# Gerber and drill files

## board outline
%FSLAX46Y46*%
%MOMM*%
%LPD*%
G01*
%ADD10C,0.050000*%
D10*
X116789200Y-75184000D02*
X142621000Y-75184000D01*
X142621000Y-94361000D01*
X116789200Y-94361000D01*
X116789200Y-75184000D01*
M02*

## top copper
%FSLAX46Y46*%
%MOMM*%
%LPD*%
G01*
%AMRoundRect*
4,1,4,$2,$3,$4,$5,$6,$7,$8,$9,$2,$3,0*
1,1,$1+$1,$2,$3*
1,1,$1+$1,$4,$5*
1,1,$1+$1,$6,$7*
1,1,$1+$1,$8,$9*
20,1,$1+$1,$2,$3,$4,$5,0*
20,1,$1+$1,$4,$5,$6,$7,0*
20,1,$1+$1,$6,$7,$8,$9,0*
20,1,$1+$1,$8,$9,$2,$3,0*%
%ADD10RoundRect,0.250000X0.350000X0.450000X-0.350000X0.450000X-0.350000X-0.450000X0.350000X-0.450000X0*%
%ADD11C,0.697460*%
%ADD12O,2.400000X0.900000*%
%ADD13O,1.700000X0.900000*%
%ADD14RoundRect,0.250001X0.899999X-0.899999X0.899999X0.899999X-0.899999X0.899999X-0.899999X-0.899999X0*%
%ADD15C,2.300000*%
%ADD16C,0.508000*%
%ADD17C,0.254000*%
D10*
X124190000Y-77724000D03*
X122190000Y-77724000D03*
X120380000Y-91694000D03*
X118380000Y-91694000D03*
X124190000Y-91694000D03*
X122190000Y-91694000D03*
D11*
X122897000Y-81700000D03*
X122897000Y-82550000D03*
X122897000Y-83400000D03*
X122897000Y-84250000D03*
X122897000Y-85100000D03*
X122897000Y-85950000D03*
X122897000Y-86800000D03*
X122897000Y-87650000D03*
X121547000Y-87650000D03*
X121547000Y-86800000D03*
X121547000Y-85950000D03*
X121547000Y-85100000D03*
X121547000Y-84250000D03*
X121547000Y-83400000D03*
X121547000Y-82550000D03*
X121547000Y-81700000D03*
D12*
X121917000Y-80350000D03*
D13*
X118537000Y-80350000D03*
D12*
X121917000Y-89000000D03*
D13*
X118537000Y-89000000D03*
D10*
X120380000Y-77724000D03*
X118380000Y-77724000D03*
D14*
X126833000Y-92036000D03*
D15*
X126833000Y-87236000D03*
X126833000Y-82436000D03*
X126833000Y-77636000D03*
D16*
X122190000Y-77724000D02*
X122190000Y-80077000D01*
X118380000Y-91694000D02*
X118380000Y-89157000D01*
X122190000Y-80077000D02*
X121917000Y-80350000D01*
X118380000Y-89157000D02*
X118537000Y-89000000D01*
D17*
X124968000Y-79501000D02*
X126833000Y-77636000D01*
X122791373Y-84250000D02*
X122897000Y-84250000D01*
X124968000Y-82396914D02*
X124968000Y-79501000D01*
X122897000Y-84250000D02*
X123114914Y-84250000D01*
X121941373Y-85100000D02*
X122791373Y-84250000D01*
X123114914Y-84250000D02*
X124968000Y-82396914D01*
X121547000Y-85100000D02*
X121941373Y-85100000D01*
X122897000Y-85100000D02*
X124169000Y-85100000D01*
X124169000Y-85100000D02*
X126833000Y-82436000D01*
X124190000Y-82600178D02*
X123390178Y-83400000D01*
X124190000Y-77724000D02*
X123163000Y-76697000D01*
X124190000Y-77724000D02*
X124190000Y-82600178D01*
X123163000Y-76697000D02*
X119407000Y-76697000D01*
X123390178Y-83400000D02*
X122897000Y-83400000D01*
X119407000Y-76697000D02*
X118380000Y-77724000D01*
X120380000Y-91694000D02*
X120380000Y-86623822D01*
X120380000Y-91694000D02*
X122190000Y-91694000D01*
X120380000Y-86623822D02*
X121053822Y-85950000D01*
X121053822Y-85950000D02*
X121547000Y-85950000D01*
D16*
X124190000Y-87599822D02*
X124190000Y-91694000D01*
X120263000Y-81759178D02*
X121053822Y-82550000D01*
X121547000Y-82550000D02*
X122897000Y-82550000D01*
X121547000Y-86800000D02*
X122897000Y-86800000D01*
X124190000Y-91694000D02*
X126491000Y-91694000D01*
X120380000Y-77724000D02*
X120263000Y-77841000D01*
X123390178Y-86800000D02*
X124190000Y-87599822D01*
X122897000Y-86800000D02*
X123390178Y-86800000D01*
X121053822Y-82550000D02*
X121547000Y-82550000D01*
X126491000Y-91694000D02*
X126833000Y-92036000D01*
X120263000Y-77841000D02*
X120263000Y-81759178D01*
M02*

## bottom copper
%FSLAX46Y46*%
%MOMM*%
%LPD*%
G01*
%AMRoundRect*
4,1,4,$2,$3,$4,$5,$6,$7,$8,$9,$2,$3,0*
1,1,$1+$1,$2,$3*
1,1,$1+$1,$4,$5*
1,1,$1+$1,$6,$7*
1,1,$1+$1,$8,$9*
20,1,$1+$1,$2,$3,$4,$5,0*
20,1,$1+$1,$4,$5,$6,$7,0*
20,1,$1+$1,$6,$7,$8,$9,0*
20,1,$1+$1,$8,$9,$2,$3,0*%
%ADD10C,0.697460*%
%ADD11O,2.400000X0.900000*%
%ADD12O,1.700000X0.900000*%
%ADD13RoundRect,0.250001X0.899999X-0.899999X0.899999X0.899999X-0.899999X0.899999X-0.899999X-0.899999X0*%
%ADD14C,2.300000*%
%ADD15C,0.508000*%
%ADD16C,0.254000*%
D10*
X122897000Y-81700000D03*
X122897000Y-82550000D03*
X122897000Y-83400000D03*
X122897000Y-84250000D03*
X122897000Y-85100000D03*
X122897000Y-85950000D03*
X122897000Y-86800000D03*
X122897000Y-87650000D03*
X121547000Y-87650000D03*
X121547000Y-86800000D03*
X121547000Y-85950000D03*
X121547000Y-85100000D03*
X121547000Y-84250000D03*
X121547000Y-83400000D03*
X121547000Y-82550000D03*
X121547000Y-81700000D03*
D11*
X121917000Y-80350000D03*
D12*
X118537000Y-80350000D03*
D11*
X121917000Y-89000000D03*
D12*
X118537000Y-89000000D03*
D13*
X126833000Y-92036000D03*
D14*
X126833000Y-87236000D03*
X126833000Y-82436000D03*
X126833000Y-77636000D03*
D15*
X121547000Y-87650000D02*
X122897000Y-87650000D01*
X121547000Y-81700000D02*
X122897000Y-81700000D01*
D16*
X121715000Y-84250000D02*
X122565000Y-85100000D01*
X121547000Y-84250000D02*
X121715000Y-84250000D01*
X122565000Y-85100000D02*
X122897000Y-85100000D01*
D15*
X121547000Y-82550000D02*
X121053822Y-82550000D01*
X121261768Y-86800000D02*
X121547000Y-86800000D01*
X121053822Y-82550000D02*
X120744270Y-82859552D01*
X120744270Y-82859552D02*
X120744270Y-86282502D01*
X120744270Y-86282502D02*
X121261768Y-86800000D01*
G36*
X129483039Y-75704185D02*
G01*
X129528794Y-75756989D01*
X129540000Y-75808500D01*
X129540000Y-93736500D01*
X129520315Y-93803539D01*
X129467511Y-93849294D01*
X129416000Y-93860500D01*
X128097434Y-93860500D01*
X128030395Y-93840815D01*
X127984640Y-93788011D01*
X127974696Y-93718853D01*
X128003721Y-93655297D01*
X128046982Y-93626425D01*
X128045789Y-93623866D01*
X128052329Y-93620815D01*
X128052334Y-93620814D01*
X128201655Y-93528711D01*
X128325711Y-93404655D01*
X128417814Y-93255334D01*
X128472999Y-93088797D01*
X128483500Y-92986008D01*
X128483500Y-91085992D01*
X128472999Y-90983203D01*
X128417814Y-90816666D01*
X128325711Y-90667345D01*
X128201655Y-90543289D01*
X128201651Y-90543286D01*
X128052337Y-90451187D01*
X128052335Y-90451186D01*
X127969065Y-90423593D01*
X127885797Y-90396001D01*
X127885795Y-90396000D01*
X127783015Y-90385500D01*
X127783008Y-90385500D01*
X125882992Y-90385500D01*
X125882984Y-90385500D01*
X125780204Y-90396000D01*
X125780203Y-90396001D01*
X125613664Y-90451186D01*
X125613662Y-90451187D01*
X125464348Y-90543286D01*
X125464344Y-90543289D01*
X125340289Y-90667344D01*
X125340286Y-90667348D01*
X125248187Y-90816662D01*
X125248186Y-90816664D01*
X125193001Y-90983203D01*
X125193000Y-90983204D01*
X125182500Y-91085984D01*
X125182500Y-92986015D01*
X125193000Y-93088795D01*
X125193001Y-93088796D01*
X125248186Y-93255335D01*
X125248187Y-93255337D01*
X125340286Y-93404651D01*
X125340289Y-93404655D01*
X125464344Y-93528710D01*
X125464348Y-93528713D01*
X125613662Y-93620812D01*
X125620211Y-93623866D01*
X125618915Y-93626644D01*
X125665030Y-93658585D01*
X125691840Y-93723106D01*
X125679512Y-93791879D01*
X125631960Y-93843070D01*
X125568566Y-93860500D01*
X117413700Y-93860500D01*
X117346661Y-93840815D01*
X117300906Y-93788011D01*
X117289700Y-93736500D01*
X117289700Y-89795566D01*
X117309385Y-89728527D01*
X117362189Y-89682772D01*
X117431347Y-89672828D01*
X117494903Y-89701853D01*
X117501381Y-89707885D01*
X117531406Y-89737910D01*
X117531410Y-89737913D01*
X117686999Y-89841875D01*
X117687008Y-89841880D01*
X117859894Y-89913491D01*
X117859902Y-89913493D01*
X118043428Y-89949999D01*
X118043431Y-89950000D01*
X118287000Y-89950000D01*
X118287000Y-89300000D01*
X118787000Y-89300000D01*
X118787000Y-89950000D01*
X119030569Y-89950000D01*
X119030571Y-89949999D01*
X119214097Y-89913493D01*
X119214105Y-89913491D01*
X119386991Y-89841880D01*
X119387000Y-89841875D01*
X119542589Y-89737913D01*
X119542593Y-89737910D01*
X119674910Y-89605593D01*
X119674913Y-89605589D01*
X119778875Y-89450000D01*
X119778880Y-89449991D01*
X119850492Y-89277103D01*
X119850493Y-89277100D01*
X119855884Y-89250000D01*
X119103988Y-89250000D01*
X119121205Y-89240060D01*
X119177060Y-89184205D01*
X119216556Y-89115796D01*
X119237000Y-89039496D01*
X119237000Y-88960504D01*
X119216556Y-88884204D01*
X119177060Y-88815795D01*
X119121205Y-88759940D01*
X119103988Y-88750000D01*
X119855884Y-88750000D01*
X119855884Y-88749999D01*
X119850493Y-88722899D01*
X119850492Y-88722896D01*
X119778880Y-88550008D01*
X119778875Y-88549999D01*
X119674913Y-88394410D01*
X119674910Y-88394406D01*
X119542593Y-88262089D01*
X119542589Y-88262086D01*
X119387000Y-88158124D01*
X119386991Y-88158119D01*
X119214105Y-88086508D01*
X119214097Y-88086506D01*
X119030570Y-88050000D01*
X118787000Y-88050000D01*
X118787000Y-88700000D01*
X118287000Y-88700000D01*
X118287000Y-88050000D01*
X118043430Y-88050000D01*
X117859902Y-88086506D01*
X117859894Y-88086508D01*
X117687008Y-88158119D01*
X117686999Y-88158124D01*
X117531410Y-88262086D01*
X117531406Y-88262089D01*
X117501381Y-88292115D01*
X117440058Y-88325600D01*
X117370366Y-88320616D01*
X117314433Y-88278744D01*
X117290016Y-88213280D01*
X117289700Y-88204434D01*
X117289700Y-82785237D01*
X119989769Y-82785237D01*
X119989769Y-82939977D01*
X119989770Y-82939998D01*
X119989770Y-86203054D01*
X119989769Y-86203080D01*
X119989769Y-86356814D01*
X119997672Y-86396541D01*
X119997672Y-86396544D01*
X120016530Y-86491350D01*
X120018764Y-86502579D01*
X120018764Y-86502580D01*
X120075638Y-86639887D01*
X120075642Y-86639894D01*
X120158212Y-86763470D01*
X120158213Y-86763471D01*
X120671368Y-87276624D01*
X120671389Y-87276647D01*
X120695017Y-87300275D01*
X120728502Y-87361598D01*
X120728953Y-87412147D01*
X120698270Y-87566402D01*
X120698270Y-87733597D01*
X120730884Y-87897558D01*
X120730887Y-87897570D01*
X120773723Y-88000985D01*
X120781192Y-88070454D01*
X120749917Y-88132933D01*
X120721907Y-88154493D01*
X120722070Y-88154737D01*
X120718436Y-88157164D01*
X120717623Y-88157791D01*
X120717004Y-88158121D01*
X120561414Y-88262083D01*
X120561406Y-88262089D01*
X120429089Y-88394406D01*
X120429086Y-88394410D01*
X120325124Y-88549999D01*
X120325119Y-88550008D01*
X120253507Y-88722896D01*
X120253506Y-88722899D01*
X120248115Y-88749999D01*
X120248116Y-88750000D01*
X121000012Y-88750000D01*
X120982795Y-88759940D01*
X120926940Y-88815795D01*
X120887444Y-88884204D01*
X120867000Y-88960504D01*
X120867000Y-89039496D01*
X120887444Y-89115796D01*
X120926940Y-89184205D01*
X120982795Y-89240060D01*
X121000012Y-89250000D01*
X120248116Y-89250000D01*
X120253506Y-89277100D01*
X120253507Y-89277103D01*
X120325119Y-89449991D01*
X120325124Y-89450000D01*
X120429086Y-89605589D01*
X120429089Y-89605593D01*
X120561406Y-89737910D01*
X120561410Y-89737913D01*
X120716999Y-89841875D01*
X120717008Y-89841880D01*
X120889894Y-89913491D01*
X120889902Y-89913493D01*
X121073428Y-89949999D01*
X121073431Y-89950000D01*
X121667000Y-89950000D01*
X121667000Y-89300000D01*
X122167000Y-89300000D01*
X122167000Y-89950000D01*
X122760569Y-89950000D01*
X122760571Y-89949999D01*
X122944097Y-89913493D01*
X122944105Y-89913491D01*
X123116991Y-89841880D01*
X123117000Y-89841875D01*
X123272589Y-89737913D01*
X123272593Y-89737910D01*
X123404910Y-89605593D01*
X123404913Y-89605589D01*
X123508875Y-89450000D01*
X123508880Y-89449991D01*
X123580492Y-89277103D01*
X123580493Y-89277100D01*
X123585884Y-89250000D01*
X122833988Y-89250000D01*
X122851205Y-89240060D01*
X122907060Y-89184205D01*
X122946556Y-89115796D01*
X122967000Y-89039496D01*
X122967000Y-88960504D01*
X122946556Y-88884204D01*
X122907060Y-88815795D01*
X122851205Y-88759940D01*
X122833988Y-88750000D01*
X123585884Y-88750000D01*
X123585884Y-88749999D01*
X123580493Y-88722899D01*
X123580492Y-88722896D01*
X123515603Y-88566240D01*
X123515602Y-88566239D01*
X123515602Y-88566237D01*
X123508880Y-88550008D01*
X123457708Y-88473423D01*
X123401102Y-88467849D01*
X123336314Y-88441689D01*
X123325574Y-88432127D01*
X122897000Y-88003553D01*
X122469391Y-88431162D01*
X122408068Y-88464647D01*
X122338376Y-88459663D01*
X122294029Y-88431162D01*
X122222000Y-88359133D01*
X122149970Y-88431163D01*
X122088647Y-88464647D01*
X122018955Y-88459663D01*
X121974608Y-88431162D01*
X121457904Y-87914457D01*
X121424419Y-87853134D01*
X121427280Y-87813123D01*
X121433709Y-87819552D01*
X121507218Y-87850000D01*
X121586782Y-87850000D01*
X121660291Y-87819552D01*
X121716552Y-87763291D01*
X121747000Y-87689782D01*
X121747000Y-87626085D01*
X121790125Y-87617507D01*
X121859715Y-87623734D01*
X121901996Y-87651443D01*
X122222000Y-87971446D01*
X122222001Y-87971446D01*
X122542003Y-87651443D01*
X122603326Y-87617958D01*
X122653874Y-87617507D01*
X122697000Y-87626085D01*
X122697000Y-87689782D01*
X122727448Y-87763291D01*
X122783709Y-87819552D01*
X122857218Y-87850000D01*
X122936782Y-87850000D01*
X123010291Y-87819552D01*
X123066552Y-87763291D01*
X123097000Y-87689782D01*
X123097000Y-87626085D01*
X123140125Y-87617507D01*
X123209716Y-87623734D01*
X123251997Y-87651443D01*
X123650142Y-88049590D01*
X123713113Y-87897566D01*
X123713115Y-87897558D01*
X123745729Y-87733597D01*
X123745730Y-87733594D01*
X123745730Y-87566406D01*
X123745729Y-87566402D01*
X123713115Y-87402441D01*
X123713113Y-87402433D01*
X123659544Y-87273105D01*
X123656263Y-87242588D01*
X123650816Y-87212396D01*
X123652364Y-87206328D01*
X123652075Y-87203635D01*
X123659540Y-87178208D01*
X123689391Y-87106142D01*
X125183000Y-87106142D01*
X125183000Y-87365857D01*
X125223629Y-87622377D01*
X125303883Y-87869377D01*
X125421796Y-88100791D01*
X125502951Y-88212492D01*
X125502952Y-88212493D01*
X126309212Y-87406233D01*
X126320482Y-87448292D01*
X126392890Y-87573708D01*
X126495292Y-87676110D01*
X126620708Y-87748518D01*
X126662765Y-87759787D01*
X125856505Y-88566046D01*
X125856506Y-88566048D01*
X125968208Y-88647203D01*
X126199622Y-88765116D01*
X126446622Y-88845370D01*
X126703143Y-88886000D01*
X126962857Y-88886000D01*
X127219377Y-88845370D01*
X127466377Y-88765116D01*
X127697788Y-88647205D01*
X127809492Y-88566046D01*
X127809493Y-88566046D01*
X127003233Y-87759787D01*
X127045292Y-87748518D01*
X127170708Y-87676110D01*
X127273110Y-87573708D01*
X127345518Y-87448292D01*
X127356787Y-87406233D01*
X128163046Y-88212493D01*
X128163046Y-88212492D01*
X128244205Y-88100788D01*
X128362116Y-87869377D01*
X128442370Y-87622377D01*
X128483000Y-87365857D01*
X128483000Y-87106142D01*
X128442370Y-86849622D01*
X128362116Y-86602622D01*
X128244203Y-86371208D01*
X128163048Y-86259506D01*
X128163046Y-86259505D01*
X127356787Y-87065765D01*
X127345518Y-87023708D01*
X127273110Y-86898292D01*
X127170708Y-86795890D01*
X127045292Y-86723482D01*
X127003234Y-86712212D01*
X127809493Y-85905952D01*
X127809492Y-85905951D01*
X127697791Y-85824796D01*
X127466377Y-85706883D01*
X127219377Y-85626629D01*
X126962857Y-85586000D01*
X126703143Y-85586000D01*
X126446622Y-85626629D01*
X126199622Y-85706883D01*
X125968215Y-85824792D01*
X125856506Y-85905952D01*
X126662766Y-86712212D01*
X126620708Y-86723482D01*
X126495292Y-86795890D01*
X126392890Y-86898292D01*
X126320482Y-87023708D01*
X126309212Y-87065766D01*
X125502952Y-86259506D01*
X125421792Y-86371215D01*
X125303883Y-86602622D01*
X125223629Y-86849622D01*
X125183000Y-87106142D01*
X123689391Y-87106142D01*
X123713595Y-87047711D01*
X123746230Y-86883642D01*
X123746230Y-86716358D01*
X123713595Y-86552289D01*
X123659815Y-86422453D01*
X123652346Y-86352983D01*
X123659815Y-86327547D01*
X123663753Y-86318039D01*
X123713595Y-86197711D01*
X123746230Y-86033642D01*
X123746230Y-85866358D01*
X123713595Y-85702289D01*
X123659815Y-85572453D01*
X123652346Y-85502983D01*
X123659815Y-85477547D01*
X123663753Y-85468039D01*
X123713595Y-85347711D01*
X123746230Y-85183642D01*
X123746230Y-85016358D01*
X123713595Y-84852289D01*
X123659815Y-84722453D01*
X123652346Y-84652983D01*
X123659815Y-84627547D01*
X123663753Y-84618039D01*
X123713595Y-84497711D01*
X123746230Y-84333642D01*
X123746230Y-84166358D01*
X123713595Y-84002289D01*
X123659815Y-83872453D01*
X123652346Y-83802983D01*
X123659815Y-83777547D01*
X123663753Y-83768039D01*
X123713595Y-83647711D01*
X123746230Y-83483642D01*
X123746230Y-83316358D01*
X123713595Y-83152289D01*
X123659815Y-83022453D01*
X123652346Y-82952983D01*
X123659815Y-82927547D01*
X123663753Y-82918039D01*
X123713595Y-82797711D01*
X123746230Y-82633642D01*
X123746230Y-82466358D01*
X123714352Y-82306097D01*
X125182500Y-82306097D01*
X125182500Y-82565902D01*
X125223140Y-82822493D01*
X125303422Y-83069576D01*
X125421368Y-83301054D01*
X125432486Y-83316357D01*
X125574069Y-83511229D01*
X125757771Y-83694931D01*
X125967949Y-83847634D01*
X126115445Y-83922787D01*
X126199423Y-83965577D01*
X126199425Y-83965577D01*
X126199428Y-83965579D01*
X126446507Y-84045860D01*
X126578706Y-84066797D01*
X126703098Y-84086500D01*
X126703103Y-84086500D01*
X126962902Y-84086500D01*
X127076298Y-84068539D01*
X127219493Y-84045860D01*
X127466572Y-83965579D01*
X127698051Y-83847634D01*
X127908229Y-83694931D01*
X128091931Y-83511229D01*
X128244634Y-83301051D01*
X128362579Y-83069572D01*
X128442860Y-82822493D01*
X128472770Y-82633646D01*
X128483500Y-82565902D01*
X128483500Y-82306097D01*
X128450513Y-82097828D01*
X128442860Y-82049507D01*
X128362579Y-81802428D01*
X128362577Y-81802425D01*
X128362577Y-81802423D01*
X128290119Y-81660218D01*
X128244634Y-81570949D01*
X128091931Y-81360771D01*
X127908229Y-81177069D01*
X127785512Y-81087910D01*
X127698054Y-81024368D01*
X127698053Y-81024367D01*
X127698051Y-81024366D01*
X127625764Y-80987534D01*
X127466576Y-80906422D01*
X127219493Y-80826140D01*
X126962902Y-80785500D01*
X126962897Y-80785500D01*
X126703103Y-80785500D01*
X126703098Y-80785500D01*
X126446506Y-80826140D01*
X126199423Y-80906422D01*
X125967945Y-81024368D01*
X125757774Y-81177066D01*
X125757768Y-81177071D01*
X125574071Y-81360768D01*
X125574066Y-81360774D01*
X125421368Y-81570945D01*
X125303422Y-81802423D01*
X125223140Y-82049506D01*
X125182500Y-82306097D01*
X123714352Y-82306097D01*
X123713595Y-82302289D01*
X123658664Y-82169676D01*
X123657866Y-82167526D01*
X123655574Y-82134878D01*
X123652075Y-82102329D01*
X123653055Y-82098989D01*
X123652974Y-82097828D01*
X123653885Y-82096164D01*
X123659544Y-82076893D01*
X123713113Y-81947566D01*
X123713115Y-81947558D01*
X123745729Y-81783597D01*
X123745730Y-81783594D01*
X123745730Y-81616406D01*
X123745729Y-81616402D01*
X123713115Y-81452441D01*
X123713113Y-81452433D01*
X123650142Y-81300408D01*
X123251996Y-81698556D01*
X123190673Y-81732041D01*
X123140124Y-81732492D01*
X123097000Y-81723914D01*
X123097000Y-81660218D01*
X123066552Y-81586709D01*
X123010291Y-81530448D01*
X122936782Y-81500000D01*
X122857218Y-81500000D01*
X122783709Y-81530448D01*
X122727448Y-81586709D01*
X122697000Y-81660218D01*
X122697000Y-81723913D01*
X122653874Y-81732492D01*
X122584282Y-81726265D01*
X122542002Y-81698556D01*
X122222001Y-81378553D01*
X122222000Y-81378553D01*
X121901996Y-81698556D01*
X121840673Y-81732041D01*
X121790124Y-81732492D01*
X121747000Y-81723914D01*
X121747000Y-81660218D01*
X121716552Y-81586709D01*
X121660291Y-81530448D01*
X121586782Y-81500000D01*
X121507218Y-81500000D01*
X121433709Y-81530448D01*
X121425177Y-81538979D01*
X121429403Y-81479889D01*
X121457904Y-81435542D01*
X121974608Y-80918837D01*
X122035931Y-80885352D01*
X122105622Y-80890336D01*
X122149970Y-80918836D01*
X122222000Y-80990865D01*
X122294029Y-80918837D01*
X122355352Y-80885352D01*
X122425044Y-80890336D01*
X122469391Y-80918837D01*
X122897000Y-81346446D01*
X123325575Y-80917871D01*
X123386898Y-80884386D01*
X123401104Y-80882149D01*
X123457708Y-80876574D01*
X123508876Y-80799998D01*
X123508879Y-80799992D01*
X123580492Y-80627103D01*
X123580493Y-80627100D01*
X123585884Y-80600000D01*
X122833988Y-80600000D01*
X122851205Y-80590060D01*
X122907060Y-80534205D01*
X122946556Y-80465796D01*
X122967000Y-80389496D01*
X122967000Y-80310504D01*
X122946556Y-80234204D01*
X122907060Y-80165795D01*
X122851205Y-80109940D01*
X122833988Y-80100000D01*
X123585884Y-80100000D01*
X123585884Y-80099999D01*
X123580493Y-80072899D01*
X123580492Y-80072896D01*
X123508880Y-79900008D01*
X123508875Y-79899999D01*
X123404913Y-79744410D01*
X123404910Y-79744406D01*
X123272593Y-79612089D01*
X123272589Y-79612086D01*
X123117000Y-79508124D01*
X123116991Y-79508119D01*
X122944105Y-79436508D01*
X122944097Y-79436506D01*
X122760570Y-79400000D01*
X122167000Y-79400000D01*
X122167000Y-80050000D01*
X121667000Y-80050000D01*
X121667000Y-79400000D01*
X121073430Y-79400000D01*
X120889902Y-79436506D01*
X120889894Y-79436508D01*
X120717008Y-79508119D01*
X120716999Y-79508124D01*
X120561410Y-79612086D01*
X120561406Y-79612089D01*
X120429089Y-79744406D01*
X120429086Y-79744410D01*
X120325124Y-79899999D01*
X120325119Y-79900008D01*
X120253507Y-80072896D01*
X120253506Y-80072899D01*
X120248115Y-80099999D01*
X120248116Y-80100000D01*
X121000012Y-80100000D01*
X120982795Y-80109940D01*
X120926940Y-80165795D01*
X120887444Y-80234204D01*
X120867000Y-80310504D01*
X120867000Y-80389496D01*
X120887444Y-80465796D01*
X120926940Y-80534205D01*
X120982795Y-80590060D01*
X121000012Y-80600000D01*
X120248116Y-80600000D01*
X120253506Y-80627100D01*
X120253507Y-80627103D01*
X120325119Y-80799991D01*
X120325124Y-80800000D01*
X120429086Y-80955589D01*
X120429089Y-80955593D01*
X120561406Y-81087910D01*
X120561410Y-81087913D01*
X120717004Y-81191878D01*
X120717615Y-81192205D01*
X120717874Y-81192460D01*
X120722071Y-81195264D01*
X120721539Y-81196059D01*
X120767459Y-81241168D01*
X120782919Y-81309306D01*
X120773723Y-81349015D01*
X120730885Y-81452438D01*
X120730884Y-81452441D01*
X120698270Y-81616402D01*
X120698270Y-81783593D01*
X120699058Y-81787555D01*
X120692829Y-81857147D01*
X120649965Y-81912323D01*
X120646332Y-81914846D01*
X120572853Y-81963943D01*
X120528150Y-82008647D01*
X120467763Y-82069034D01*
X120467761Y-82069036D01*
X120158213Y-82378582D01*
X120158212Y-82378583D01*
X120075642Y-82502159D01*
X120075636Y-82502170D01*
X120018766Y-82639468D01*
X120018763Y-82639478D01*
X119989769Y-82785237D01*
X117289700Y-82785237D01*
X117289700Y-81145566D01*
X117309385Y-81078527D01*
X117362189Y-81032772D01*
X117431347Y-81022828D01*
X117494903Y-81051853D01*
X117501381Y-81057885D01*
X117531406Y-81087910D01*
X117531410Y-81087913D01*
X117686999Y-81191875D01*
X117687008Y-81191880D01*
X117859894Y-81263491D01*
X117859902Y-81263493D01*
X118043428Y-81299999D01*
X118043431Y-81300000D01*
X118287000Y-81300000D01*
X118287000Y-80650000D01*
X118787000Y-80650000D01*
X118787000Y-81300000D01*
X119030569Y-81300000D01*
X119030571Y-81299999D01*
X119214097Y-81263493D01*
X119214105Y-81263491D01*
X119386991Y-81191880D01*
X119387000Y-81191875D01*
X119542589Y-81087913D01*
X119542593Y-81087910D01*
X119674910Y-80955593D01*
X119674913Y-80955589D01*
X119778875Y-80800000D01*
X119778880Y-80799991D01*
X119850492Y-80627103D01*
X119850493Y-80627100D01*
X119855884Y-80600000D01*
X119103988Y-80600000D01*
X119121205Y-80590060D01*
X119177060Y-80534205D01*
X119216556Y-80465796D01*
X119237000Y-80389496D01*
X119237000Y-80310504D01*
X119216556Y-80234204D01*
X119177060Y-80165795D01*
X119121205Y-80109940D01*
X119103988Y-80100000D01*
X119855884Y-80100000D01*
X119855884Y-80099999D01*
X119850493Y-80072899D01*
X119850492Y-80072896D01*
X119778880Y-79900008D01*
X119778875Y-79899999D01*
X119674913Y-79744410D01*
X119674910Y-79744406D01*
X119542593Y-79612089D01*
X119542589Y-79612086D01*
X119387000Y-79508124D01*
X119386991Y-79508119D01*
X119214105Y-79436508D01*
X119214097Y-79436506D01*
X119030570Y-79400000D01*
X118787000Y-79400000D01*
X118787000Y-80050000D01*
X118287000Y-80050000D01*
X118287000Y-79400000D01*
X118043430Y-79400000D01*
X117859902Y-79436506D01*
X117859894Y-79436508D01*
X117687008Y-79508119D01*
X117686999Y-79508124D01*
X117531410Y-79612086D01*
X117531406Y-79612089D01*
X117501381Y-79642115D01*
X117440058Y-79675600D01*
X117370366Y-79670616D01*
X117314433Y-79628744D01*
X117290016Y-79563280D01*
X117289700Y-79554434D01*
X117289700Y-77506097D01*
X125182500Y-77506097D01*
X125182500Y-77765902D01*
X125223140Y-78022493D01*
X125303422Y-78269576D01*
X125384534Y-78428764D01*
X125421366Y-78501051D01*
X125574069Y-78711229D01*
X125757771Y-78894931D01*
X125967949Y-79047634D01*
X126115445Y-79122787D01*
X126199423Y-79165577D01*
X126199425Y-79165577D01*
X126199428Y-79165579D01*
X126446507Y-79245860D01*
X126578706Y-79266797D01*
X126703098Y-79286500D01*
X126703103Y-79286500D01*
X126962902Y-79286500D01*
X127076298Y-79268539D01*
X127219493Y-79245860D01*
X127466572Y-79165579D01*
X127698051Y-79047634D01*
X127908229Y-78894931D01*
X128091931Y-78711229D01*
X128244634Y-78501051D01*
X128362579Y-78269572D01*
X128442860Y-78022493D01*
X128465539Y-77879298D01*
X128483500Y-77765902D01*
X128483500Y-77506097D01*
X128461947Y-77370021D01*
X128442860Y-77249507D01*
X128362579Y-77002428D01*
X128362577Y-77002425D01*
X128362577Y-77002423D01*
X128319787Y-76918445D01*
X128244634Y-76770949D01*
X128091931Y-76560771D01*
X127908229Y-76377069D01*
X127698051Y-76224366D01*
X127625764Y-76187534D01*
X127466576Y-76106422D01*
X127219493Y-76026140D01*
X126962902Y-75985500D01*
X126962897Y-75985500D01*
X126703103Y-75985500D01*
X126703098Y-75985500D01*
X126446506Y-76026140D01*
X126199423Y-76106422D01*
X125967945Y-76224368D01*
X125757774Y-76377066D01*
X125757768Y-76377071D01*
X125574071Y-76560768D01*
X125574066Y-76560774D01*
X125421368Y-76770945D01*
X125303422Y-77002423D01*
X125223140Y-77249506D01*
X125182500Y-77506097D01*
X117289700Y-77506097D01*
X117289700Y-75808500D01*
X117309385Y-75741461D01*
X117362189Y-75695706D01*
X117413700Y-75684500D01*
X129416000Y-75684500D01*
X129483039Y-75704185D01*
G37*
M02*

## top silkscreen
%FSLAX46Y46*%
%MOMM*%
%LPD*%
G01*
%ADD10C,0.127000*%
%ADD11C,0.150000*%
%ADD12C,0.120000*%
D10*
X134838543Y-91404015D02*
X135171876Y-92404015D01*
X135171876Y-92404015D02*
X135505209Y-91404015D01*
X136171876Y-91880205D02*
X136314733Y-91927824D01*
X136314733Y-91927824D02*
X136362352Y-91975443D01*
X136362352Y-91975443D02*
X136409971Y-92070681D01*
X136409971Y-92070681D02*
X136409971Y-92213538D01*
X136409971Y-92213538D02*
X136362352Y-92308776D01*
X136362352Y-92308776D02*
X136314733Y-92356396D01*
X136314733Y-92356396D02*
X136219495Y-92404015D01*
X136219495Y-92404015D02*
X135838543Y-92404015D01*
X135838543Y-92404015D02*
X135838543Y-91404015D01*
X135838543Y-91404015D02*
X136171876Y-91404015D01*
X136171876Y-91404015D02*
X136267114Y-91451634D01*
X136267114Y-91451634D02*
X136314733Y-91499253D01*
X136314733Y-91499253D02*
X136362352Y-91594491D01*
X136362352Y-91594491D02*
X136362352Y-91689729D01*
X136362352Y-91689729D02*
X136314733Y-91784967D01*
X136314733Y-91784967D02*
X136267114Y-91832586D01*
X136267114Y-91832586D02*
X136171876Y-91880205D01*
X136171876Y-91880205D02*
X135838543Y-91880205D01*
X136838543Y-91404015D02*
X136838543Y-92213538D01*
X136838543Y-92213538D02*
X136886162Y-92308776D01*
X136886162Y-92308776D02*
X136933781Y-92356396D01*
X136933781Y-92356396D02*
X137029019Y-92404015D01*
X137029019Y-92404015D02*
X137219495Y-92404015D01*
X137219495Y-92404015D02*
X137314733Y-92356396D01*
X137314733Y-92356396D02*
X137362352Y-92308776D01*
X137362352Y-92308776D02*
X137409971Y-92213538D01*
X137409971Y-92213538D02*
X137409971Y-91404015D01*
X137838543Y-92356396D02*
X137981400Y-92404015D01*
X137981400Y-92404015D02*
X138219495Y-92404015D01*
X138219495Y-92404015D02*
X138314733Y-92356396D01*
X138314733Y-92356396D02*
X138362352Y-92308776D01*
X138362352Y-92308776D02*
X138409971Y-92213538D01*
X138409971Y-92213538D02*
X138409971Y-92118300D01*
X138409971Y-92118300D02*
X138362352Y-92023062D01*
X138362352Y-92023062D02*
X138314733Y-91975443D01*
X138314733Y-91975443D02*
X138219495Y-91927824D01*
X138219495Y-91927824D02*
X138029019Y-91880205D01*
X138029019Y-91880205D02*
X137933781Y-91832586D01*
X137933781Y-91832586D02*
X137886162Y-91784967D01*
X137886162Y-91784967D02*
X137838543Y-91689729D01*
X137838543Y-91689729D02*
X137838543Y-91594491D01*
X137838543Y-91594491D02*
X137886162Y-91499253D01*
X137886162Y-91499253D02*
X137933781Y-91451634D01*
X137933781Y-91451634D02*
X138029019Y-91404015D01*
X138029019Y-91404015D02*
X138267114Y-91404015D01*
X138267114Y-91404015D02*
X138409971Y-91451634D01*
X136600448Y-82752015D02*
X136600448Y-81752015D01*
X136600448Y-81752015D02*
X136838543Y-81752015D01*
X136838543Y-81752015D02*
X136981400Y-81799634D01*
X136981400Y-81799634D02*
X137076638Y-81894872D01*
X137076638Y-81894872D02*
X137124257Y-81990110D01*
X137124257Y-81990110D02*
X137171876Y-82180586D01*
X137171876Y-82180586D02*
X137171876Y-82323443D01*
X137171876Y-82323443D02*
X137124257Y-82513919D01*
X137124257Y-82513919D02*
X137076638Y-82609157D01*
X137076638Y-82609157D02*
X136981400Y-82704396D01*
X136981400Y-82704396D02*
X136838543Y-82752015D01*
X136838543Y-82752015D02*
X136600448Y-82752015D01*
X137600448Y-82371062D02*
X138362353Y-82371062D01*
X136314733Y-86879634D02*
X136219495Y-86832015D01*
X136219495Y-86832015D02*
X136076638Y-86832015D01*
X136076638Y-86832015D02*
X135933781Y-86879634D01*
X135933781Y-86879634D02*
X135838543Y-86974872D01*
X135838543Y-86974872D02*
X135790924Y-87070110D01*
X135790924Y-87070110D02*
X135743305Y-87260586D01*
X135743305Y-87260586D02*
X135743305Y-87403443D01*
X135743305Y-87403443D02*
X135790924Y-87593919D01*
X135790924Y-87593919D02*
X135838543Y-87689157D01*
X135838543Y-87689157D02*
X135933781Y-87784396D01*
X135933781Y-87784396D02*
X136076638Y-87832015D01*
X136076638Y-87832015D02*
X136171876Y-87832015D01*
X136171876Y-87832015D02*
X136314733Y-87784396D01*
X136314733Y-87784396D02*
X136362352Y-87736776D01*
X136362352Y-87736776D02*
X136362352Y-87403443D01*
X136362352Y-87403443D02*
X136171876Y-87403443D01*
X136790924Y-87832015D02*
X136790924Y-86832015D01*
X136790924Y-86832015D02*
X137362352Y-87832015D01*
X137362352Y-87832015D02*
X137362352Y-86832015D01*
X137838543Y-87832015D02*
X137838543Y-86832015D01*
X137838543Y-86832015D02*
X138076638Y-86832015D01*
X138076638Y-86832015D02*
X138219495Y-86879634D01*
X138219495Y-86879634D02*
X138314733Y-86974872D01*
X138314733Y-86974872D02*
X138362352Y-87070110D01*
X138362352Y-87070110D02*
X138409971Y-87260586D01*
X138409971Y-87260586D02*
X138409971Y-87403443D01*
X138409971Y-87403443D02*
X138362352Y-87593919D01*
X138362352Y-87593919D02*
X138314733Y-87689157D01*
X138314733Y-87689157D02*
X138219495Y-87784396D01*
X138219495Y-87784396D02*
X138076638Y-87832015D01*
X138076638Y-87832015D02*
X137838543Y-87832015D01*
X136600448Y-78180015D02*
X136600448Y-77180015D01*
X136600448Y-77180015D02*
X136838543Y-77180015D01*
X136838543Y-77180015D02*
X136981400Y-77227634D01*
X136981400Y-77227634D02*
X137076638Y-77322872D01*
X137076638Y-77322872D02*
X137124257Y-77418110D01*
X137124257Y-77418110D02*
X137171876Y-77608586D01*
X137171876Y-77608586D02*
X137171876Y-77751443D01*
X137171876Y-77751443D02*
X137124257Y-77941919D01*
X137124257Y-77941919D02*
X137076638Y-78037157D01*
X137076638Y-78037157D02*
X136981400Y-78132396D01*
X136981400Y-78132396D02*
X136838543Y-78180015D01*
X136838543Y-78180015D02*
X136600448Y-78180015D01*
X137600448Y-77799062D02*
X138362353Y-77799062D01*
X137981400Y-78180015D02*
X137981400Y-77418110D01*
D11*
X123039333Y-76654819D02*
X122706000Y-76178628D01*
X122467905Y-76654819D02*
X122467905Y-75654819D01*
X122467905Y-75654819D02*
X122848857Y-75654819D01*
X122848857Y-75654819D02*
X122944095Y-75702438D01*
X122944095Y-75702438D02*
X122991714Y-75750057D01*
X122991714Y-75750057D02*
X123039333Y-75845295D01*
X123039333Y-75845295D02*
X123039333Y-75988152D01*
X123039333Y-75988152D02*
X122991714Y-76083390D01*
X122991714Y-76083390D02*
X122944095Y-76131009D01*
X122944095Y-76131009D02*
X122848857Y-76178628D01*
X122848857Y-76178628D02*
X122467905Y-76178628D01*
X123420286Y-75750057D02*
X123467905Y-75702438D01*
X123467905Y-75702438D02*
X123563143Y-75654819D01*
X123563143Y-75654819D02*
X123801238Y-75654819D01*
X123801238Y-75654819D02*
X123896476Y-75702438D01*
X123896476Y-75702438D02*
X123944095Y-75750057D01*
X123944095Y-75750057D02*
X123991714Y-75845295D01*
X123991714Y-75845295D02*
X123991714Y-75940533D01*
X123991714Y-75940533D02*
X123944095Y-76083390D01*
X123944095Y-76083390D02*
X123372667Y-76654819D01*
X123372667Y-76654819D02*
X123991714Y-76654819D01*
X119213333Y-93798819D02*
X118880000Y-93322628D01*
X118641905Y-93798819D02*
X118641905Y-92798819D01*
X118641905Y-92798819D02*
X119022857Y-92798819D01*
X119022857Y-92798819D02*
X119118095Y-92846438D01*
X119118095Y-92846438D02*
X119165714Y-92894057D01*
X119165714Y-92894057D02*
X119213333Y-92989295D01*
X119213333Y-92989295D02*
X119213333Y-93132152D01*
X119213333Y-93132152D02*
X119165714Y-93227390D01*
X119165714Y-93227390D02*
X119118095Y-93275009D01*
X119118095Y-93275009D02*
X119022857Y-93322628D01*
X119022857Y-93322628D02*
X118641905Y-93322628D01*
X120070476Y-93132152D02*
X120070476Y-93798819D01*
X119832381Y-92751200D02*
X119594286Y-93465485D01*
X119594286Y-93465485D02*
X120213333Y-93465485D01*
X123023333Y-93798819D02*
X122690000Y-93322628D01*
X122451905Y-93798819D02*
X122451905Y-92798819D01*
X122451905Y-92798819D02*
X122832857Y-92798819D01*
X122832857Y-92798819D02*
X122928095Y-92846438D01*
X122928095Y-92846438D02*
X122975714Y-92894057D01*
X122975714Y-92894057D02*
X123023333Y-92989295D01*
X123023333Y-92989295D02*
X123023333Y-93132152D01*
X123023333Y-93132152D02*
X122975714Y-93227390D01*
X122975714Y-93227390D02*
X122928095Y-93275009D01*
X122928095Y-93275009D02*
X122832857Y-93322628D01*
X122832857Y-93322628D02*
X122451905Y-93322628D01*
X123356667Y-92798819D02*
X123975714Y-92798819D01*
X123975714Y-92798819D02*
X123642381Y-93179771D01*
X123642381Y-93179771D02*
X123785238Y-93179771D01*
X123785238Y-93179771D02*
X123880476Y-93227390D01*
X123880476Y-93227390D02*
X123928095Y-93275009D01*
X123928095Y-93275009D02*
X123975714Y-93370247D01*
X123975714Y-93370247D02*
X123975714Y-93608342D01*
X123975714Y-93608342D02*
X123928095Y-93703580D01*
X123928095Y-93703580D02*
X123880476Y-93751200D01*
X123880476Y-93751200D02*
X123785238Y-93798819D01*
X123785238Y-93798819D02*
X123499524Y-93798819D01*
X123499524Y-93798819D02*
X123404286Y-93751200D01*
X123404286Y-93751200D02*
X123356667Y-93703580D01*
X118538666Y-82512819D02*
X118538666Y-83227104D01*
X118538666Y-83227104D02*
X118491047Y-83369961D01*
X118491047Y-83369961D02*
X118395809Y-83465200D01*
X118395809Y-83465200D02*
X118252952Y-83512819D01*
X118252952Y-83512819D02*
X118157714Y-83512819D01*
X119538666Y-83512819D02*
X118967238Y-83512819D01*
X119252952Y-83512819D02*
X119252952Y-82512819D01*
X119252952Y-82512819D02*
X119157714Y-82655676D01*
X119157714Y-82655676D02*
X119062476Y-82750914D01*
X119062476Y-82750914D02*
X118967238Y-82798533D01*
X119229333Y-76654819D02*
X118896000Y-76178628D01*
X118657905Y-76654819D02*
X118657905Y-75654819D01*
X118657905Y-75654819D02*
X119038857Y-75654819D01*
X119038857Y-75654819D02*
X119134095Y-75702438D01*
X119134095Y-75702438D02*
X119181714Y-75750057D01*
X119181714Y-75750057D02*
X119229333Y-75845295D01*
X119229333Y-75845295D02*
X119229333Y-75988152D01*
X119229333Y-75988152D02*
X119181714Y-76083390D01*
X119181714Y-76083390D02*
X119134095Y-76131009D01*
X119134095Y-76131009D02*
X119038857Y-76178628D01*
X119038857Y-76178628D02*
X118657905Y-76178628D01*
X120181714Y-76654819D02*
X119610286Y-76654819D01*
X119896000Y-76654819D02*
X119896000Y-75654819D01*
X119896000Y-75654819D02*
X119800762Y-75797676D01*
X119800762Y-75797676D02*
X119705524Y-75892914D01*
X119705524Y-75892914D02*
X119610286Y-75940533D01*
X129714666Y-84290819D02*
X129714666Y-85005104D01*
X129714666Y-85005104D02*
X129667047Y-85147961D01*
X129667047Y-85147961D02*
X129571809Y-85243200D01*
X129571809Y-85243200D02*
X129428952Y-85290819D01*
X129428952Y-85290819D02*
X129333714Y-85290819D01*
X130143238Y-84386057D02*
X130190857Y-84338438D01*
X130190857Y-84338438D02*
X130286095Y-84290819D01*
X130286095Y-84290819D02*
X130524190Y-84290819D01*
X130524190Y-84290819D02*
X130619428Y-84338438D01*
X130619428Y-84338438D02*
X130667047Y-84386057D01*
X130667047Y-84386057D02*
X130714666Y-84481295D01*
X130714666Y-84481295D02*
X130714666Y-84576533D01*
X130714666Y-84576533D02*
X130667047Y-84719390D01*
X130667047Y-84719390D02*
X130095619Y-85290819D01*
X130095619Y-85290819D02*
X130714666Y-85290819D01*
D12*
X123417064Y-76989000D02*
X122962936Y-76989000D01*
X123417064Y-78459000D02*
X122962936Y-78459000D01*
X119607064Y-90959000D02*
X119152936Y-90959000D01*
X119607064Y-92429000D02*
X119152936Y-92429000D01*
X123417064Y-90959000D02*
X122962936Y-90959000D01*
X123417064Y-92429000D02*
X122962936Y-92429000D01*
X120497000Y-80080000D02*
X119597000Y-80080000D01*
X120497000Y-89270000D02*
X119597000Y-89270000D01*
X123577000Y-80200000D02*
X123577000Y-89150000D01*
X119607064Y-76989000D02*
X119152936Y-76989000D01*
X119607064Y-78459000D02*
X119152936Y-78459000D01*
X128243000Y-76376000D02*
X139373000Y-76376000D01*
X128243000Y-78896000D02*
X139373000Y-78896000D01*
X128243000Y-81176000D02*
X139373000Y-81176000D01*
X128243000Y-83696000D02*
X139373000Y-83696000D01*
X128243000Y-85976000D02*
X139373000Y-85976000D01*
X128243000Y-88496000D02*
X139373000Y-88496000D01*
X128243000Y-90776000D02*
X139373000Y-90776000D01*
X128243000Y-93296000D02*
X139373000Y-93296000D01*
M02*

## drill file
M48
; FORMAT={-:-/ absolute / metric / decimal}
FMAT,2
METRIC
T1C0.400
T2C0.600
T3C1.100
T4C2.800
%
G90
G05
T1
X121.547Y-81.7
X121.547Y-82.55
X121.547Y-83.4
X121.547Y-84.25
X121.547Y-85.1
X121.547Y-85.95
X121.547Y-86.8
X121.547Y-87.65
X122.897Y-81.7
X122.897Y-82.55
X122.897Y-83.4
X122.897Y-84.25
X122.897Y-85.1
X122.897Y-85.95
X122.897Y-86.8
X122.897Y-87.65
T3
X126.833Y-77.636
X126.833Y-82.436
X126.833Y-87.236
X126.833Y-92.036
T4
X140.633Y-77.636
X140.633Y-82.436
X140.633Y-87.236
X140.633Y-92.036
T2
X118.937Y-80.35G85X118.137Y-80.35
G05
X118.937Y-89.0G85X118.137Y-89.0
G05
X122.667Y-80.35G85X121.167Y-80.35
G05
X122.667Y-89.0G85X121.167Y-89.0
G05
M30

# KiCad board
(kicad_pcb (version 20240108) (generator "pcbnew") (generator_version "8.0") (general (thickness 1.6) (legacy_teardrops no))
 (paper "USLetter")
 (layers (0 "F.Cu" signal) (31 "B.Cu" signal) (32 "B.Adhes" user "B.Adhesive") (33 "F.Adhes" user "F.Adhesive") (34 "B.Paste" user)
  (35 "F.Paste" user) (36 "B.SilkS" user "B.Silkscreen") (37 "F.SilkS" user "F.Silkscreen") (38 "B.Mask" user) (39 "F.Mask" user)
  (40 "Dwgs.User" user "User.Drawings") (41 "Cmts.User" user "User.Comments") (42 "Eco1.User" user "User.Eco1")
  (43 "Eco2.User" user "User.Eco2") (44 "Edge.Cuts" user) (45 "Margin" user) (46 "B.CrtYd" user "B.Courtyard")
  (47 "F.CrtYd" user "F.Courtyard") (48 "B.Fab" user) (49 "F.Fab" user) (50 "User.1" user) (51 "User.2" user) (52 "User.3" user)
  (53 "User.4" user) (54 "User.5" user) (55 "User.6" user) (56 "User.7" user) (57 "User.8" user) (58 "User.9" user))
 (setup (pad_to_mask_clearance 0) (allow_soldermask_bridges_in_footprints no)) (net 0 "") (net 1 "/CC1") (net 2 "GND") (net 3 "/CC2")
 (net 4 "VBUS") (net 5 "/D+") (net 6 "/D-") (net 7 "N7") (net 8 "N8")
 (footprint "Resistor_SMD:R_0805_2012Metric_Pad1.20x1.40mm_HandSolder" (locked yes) (layer "F.Cu") (at 123.19 77.724 180)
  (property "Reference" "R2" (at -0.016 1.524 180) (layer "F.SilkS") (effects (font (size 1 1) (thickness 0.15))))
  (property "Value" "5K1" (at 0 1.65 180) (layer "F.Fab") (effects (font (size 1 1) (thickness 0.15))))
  (fp_line (start -0.227064 0.735) (end 0.227064 0.735) (stroke (width 0.12) (type solid)) (layer "F.SilkS"))
  (fp_line (start -0.227064 -0.735) (end 0.227064 -0.735) (stroke (width 0.12) (type solid)) (layer "F.SilkS"))
  (pad "1" smd roundrect (at -1 0 180) (size 1.2 1.4) (layers "F.Cu" "F.Paste" "F.Mask") (roundrect_rratio 0.208333) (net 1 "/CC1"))
  (pad "2" smd roundrect (at 1 0 180) (size 1.2 1.4) (layers "F.Cu" "F.Paste" "F.Mask") (roundrect_rratio 0.208333) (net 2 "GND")))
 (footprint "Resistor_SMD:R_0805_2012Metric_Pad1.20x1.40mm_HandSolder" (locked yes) (layer "F.Cu") (at 119.38 91.694 180)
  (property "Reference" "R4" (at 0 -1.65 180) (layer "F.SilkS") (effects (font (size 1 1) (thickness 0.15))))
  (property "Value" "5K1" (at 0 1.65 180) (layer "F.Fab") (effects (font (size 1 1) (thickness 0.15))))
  (fp_line (start -0.227064 0.735) (end 0.227064 0.735) (stroke (width 0.12) (type solid)) (layer "F.SilkS"))
  (fp_line (start -0.227064 -0.735) (end 0.227064 -0.735) (stroke (width 0.12) (type solid)) (layer "F.SilkS"))
  (pad "1" smd roundrect (at -1 0 180) (size 1.2 1.4) (layers "F.Cu" "F.Paste" "F.Mask") (roundrect_rratio 0.208333) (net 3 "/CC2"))
  (pad "2" smd roundrect (at 1 0 180) (size 1.2 1.4) (layers "F.Cu" "F.Paste" "F.Mask") (roundrect_rratio 0.208333) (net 2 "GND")))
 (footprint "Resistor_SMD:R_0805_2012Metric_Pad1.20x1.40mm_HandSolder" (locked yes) (layer "F.Cu") (at 123.19 91.694 180)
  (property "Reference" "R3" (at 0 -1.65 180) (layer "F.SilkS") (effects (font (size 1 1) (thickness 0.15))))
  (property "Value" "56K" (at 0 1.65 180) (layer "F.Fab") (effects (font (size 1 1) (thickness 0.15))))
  (fp_line (start -0.227064 0.735) (end 0.227064 0.735) (stroke (width 0.12) (type solid)) (layer "F.SilkS"))
  (fp_line (start -0.227064 -0.735) (end 0.227064 -0.735) (stroke (width 0.12) (type solid)) (layer "F.SilkS"))
  (pad "1" smd roundrect (at -1 0 180) (size 1.2 1.4) (layers "F.Cu" "F.Paste" "F.Mask") (roundrect_rratio 0.208333) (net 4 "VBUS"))
  (pad "2" smd roundrect (at 1 0 180) (size 1.2 1.4) (layers "F.Cu" "F.Paste" "F.Mask") (roundrect_rratio 0.208333) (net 3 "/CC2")))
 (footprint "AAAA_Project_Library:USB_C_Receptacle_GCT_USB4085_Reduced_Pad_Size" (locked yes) (layer "F.Cu") (at 122.897 81.7 -90)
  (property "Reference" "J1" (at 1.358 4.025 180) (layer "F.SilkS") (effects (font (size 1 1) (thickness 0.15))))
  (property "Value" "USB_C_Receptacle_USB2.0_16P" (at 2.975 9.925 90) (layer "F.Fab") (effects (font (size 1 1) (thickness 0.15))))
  (fp_line (start -1.62 2.4) (end -1.62 3.3) (stroke (width 0.12) (type solid)) (layer "F.SilkS"))
  (fp_line (start 7.57 2.4) (end 7.57 3.3) (stroke (width 0.12) (type solid)) (layer "F.SilkS"))
  (fp_line (start -1.5 -0.68) (end 7.45 -0.68) (stroke (width 0.12) (type solid)) (layer "F.SilkS"))
  (pad "A1" thru_hole circle (at 0 0 270) (size 0.69746 0.69746) (drill 0.4) (layers "*.Cu" "*.Mask") (remove_unused_layers no)
   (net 2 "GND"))
  (pad "A4" thru_hole circle (at 0.85 0 270) (size 0.69746 0.69746) (drill 0.4) (layers "*.Cu" "*.Mask") (remove_unused_layers no)
   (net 4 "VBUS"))
  (pad "A5" thru_hole circle (at 1.7 0 270) (size 0.69746 0.69746) (drill 0.4) (layers "*.Cu" "*.Mask") (remove_unused_layers no)
   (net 1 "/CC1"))
  (pad "A6" thru_hole circle (at 2.55 0 270) (size 0.69746 0.69746) (drill 0.4) (layers "*.Cu" "*.Mask") (remove_unused_layers no)
   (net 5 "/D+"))
  (pad "A7" thru_hole circle (at 3.4 0 270) (size 0.69746 0.69746) (drill 0.4) (layers "*.Cu" "*.Mask") (remove_unused_layers no)
   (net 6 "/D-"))
  (pad "A8" thru_hole circle (at 4.25 0 270) (size 0.69746 0.69746) (drill 0.4) (layers "*.Cu" "*.Mask") (remove_unused_layers no)
   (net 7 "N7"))
  (pad "A9" thru_hole circle (at 5.1 0 270) (size 0.69746 0.69746) (drill 0.4) (layers "*.Cu" "*.Mask") (remove_unused_layers no)
   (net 4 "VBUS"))
  (pad "A12" thru_hole circle (at 5.95 0 270) (size 0.69746 0.69746) (drill 0.4) (layers "*.Cu" "*.Mask") (remove_unused_layers no)
   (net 2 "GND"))
  (pad "B1" thru_hole circle (at 5.95 1.35 270) (size 0.69746 0.69746) (drill 0.4) (layers "*.Cu" "*.Mask") (remove_unused_layers no)
   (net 2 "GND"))
  (pad "B4" thru_hole circle (at 5.1 1.35 270) (size 0.69746 0.69746) (drill 0.4) (layers "*.Cu" "*.Mask") (remove_unused_layers no)
   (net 4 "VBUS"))
  (pad "B5" thru_hole circle (at 4.25 1.35 270) (size 0.69746 0.69746) (drill 0.4) (layers "*.Cu" "*.Mask") (remove_unused_layers no)
   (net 3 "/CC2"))
  (pad "B6" thru_hole circle (at 3.4 1.35 270) (size 0.69746 0.69746) (drill 0.4) (layers "*.Cu" "*.Mask") (remove_unused_layers no)
   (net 5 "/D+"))
  (pad "B7" thru_hole circle (at 2.55 1.35 270) (size 0.69746 0.69746) (drill 0.4) (layers "*.Cu" "*.Mask") (remove_unused_layers no)
   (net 6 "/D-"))
  (pad "B8" thru_hole circle (at 1.7 1.35 270) (size 0.69746 0.69746) (drill 0.4) (layers "*.Cu" "*.Mask") (remove_unused_layers no)
   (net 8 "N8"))
  (pad "B9" thru_hole circle (at 0.85 1.35 270) (size 0.69746 0.69746) (drill 0.4) (layers "*.Cu" "*.Mask") (remove_unused_layers no)
   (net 4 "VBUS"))
  (pad "B12" thru_hole circle (at 0 1.35 270) (size 0.69746 0.69746) (drill 0.4) (layers "*.Cu" "*.Mask") (remove_unused_layers no)
   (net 2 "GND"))
  (pad "S1" thru_hole oval (at -1.35 0.98 270) (size 0.9 2.4) (drill oval 0.6 2.1) (layers "*.Cu" "*.Mask") (remove_unused_layers no)
   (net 2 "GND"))
  (pad "S1" thru_hole oval (at -1.35 4.36 270) (size 0.9 1.7) (drill oval 0.6 1.4) (layers "*.Cu" "*.Mask") (remove_unused_layers no)
   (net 2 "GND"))
  (pad "S1" thru_hole oval (at 7.3 0.98 270) (size 0.9 2.4) (drill oval 0.6 2.1) (layers "*.Cu" "*.Mask") (remove_unused_layers no)
   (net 2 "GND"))
  (pad "S1" thru_hole oval (at 7.3 4.36 270) (size 0.9 1.7) (drill oval 0.6 1.4) (layers "*.Cu" "*.Mask") (remove_unused_layers no)
   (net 2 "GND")))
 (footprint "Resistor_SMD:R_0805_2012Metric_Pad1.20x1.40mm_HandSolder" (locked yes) (layer "F.Cu") (at 119.38 77.724 180)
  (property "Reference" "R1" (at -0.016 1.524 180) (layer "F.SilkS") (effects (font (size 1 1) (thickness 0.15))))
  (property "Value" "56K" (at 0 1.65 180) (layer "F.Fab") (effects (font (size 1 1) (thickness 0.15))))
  (fp_line (start -0.227064 0.735) (end 0.227064 0.735) (stroke (width 0.12) (type solid)) (layer "F.SilkS"))
  (fp_line (start -0.227064 -0.735) (end 0.227064 -0.735) (stroke (width 0.12) (type solid)) (layer "F.SilkS"))
  (pad "1" smd roundrect (at -1 0 180) (size 1.2 1.4) (layers "F.Cu" "F.Paste" "F.Mask") (roundrect_rratio 0.208333) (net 4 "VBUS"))
  (pad "2" smd roundrect (at 1 0 180) (size 1.2 1.4) (layers "F.Cu" "F.Paste" "F.Mask") (roundrect_rratio 0.208333) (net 1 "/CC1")))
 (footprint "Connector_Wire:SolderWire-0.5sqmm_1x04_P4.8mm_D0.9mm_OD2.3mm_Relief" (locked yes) (layer "F.Cu") (at 126.833 92.036 90)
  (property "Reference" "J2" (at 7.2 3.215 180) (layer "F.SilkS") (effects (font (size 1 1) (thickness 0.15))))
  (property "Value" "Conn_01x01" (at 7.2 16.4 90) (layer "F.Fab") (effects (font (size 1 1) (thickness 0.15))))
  (fp_line (start 15.66 1.41) (end 15.66 12.54) (stroke (width 0.12) (type solid)) (layer "F.SilkS"))
  (fp_line (start 13.14 1.41) (end 13.14 12.54) (stroke (width 0.12) (type solid)) (layer "F.SilkS"))
  (fp_line (start 10.86 1.41) (end 10.86 12.54) (stroke (width 0.12) (type solid)) (layer "F.SilkS"))
  (fp_line (start 8.34 1.41) (end 8.34 12.54) (stroke (width 0.12) (type solid)) (layer "F.SilkS"))
  (fp_line (start 6.06 1.41) (end 6.06 12.54) (stroke (width 0.12) (type solid)) (layer "F.SilkS"))
  (fp_line (start 3.54 1.41) (end 3.54 12.54) (stroke (width 0.12) (type solid)) (layer "F.SilkS"))
  (fp_line (start 1.26 1.41) (end 1.26 12.54) (stroke (width 0.12) (type solid)) (layer "F.SilkS"))
  (fp_line (start -1.26 1.41) (end -1.26 12.54) (stroke (width 0.12) (type solid)) (layer "F.SilkS"))
  (pad "" np_thru_hole circle (at 0 13.8 90) (size 2.8 2.8) (drill 2.8) (layers "*.Cu" "*.Mask"))
  (pad "" np_thru_hole circle (at 4.8 13.8 90) (size 2.8 2.8) (drill 2.8) (layers "*.Cu" "*.Mask"))
  (pad "" np_thru_hole circle (at 9.6 13.8 90) (size 2.8 2.8) (drill 2.8) (layers "*.Cu" "*.Mask"))
  (pad "" np_thru_hole circle (at 14.4 13.8 90) (size 2.8 2.8) (drill 2.8) (layers "*.Cu" "*.Mask"))
  (pad "1" thru_hole roundrect (at 0 0 90) (size 2.3 2.3) (drill 1.1) (layers "*.Cu" "*.Mask") (remove_unused_layers no)
   (roundrect_rratio 0.108696) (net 4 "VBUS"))
  (pad "2" thru_hole circle (at 4.8 0 90) (size 2.3 2.3) (drill 1.1) (layers "*.Cu" "*.Mask") (remove_unused_layers no) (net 2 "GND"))
  (pad "3" thru_hole circle (at 9.6 0 90) (size 2.3 2.3) (drill 1.1) (layers "*.Cu" "*.Mask") (remove_unused_layers no) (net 6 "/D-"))
  (pad "4" thru_hole circle (at 14.4 0 90) (size 2.3 2.3) (drill 1.1) (layers "*.Cu" "*.Mask") (remove_unused_layers no) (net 5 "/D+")))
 (gr_rect (start 116.7892 75.184) (end 142.621 94.361) (locked yes) (stroke (width 0.05) (type default)) (fill none) (layer "Edge.Cuts"))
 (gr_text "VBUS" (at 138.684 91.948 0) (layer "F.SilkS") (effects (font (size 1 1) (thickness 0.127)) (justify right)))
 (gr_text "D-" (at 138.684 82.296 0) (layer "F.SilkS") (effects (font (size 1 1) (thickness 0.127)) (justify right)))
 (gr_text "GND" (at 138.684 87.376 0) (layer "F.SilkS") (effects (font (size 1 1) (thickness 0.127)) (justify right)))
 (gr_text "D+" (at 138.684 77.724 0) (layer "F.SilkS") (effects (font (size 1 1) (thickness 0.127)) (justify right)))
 (segment (start 122.19 77.724) (end 122.19 80.077) (width 0.508) (layer "F.Cu") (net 2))
 (segment (start 118.38 91.694) (end 118.38 89.157) (width 0.508) (layer "F.Cu") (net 2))
 (segment (start 122.19 80.077) (end 121.917 80.35) (width 0.508) (layer "F.Cu") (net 2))
 (segment (start 118.38 89.157) (end 118.537 89) (width 0.508) (layer "F.Cu") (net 2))
 (segment (start 121.547 87.65) (end 122.897 87.65) (width 0.508) (layer "B.Cu") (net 2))
 (segment (start 121.547 81.7) (end 122.897 81.7) (width 0.508) (layer "B.Cu") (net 2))
 (segment (start 124.968 79.501) (end 126.833 77.636) (width 0.254) (layer "F.Cu") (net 5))
 (segment (start 122.791373 84.25) (end 122.897 84.25) (width 0.254) (locked yes) (layer "F.Cu") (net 5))
 (segment (start 124.968 82.396914) (end 124.968 79.501) (width 0.254) (layer "F.Cu") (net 5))
 (segment (start 122.897 84.25) (end 123.114914 84.25) (width 0.254) (layer "F.Cu") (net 5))
 (segment (start 121.941373 85.1) (end 122.791373 84.25) (width 0.254) (locked yes) (layer "F.Cu") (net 5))
 (segment (start 123.114914 84.25) (end 124.968 82.396914) (width 0.254) (layer "F.Cu") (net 5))
 (segment (start 121.547 85.1) (end 121.941373 85.1) (width 0.254) (locked yes) (layer "F.Cu") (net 5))
 (segment (start 122.897 85.1) (end 124.169 85.1) (width 0.254) (layer "F.Cu") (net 6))
 (segment (start 124.169 85.1) (end 126.833 82.436) (width 0.254) (layer "F.Cu") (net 6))
 (segment (start 121.715 84.25) (end 122.565 85.1) (width 0.254) (locked yes) (layer "B.Cu") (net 6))
 (segment (start 121.547 84.25) (end 121.715 84.25) (width 0.254) (locked yes) (layer "B.Cu") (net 6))
 (segment (start 122.565 85.1) (end 122.897 85.1) (width 0.254) (locked yes) (layer "B.Cu") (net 6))
 (segment (start 124.19 82.600178) (end 123.390178 83.4) (width 0.254) (layer "F.Cu") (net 1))
 (segment (start 124.19 77.724) (end 123.163 76.697) (width 0.254) (layer "F.Cu") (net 1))
 (segment (start 124.19 77.724) (end 124.19 82.600178) (width 0.254) (layer "F.Cu") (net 1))
 (segment (start 123.163 76.697) (end 119.407 76.697) (width 0.254) (layer "F.Cu") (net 1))
 (segment (start 123.390178 83.4) (end 122.897 83.4) (width 0.254) (layer "F.Cu") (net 1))
 (segment (start 119.407 76.697) (end 118.38 77.724) (width 0.254) (layer "F.Cu") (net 1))
 (segment (start 120.38 91.694) (end 120.38 86.623822) (width 0.254) (layer "F.Cu") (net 3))
 (segment (start 120.38 91.694) (end 122.19 91.694) (width 0.254) (layer "F.Cu") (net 3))
 (segment (start 120.38 86.623822) (end 121.053822 85.95) (width 0.254) (layer "F.Cu") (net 3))
 (segment (start 121.053822 85.95) (end 121.547 85.95) (width 0.254) (layer "F.Cu") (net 3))
 (segment (start 124.19 87.599822) (end 124.19 91.694) (width 0.508) (layer "F.Cu") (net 4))
 (segment (start 120.263 81.759178) (end 121.053822 82.55) (width 0.508) (layer "F.Cu") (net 4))
 (segment (start 121.547 82.55) (end 122.897 82.55) (width 0.508) (locked yes) (layer "F.Cu") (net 4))
 (segment (start 121.547 86.8) (end 122.897 86.8) (width 0.508) (locked yes) (layer "F.Cu") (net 4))
 (segment (start 124.19 91.694) (end 126.491 91.694) (width 0.508) (layer "F.Cu") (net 4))
 (segment (start 120.38 77.724) (end 120.263 77.841) (width 0.508) (layer "F.Cu") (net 4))
 (segment (start 123.390178 86.8) (end 124.19 87.599822) (width 0.508) (layer "F.Cu") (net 4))
 (segment (start 122.897 86.8) (end 123.390178 86.8) (width 0.508) (layer "F.Cu") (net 4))
 (segment (start 121.053822 82.55) (end 121.547 82.55) (width 0.508) (layer "F.Cu") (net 4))
 (segment (start 126.491 91.694) (end 126.833 92.036) (width 0.508) (layer "F.Cu") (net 4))
 (segment (start 120.263 77.841) (end 120.263 81.759178) (width 0.508) (layer "F.Cu") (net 4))
 (segment (start 121.547 82.55) (end 121.053822 82.55) (width 0.508) (locked yes) (layer "B.Cu") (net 4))
 (segment (start 121.261768 86.8) (end 121.547 86.8) (width 0.508) (locked yes) (layer "B.Cu") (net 4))
 (segment (start 121.053822 82.55) (end 120.74427 82.859552) (width 0.508) (locked yes) (layer "B.Cu") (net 4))
 (segment (start 120.74427 82.859552) (end 120.74427 86.282502) (width 0.508) (locked yes) (layer "B.Cu") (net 4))
 (segment (start 120.74427 86.282502) (end 121.261768 86.8) (width 0.508) (locked yes) (layer "B.Cu") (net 4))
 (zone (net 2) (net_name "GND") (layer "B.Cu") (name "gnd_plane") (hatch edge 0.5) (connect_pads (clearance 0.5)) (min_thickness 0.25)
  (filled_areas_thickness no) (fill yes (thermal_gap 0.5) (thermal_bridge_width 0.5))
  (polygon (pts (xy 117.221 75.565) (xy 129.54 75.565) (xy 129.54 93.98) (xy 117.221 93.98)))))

